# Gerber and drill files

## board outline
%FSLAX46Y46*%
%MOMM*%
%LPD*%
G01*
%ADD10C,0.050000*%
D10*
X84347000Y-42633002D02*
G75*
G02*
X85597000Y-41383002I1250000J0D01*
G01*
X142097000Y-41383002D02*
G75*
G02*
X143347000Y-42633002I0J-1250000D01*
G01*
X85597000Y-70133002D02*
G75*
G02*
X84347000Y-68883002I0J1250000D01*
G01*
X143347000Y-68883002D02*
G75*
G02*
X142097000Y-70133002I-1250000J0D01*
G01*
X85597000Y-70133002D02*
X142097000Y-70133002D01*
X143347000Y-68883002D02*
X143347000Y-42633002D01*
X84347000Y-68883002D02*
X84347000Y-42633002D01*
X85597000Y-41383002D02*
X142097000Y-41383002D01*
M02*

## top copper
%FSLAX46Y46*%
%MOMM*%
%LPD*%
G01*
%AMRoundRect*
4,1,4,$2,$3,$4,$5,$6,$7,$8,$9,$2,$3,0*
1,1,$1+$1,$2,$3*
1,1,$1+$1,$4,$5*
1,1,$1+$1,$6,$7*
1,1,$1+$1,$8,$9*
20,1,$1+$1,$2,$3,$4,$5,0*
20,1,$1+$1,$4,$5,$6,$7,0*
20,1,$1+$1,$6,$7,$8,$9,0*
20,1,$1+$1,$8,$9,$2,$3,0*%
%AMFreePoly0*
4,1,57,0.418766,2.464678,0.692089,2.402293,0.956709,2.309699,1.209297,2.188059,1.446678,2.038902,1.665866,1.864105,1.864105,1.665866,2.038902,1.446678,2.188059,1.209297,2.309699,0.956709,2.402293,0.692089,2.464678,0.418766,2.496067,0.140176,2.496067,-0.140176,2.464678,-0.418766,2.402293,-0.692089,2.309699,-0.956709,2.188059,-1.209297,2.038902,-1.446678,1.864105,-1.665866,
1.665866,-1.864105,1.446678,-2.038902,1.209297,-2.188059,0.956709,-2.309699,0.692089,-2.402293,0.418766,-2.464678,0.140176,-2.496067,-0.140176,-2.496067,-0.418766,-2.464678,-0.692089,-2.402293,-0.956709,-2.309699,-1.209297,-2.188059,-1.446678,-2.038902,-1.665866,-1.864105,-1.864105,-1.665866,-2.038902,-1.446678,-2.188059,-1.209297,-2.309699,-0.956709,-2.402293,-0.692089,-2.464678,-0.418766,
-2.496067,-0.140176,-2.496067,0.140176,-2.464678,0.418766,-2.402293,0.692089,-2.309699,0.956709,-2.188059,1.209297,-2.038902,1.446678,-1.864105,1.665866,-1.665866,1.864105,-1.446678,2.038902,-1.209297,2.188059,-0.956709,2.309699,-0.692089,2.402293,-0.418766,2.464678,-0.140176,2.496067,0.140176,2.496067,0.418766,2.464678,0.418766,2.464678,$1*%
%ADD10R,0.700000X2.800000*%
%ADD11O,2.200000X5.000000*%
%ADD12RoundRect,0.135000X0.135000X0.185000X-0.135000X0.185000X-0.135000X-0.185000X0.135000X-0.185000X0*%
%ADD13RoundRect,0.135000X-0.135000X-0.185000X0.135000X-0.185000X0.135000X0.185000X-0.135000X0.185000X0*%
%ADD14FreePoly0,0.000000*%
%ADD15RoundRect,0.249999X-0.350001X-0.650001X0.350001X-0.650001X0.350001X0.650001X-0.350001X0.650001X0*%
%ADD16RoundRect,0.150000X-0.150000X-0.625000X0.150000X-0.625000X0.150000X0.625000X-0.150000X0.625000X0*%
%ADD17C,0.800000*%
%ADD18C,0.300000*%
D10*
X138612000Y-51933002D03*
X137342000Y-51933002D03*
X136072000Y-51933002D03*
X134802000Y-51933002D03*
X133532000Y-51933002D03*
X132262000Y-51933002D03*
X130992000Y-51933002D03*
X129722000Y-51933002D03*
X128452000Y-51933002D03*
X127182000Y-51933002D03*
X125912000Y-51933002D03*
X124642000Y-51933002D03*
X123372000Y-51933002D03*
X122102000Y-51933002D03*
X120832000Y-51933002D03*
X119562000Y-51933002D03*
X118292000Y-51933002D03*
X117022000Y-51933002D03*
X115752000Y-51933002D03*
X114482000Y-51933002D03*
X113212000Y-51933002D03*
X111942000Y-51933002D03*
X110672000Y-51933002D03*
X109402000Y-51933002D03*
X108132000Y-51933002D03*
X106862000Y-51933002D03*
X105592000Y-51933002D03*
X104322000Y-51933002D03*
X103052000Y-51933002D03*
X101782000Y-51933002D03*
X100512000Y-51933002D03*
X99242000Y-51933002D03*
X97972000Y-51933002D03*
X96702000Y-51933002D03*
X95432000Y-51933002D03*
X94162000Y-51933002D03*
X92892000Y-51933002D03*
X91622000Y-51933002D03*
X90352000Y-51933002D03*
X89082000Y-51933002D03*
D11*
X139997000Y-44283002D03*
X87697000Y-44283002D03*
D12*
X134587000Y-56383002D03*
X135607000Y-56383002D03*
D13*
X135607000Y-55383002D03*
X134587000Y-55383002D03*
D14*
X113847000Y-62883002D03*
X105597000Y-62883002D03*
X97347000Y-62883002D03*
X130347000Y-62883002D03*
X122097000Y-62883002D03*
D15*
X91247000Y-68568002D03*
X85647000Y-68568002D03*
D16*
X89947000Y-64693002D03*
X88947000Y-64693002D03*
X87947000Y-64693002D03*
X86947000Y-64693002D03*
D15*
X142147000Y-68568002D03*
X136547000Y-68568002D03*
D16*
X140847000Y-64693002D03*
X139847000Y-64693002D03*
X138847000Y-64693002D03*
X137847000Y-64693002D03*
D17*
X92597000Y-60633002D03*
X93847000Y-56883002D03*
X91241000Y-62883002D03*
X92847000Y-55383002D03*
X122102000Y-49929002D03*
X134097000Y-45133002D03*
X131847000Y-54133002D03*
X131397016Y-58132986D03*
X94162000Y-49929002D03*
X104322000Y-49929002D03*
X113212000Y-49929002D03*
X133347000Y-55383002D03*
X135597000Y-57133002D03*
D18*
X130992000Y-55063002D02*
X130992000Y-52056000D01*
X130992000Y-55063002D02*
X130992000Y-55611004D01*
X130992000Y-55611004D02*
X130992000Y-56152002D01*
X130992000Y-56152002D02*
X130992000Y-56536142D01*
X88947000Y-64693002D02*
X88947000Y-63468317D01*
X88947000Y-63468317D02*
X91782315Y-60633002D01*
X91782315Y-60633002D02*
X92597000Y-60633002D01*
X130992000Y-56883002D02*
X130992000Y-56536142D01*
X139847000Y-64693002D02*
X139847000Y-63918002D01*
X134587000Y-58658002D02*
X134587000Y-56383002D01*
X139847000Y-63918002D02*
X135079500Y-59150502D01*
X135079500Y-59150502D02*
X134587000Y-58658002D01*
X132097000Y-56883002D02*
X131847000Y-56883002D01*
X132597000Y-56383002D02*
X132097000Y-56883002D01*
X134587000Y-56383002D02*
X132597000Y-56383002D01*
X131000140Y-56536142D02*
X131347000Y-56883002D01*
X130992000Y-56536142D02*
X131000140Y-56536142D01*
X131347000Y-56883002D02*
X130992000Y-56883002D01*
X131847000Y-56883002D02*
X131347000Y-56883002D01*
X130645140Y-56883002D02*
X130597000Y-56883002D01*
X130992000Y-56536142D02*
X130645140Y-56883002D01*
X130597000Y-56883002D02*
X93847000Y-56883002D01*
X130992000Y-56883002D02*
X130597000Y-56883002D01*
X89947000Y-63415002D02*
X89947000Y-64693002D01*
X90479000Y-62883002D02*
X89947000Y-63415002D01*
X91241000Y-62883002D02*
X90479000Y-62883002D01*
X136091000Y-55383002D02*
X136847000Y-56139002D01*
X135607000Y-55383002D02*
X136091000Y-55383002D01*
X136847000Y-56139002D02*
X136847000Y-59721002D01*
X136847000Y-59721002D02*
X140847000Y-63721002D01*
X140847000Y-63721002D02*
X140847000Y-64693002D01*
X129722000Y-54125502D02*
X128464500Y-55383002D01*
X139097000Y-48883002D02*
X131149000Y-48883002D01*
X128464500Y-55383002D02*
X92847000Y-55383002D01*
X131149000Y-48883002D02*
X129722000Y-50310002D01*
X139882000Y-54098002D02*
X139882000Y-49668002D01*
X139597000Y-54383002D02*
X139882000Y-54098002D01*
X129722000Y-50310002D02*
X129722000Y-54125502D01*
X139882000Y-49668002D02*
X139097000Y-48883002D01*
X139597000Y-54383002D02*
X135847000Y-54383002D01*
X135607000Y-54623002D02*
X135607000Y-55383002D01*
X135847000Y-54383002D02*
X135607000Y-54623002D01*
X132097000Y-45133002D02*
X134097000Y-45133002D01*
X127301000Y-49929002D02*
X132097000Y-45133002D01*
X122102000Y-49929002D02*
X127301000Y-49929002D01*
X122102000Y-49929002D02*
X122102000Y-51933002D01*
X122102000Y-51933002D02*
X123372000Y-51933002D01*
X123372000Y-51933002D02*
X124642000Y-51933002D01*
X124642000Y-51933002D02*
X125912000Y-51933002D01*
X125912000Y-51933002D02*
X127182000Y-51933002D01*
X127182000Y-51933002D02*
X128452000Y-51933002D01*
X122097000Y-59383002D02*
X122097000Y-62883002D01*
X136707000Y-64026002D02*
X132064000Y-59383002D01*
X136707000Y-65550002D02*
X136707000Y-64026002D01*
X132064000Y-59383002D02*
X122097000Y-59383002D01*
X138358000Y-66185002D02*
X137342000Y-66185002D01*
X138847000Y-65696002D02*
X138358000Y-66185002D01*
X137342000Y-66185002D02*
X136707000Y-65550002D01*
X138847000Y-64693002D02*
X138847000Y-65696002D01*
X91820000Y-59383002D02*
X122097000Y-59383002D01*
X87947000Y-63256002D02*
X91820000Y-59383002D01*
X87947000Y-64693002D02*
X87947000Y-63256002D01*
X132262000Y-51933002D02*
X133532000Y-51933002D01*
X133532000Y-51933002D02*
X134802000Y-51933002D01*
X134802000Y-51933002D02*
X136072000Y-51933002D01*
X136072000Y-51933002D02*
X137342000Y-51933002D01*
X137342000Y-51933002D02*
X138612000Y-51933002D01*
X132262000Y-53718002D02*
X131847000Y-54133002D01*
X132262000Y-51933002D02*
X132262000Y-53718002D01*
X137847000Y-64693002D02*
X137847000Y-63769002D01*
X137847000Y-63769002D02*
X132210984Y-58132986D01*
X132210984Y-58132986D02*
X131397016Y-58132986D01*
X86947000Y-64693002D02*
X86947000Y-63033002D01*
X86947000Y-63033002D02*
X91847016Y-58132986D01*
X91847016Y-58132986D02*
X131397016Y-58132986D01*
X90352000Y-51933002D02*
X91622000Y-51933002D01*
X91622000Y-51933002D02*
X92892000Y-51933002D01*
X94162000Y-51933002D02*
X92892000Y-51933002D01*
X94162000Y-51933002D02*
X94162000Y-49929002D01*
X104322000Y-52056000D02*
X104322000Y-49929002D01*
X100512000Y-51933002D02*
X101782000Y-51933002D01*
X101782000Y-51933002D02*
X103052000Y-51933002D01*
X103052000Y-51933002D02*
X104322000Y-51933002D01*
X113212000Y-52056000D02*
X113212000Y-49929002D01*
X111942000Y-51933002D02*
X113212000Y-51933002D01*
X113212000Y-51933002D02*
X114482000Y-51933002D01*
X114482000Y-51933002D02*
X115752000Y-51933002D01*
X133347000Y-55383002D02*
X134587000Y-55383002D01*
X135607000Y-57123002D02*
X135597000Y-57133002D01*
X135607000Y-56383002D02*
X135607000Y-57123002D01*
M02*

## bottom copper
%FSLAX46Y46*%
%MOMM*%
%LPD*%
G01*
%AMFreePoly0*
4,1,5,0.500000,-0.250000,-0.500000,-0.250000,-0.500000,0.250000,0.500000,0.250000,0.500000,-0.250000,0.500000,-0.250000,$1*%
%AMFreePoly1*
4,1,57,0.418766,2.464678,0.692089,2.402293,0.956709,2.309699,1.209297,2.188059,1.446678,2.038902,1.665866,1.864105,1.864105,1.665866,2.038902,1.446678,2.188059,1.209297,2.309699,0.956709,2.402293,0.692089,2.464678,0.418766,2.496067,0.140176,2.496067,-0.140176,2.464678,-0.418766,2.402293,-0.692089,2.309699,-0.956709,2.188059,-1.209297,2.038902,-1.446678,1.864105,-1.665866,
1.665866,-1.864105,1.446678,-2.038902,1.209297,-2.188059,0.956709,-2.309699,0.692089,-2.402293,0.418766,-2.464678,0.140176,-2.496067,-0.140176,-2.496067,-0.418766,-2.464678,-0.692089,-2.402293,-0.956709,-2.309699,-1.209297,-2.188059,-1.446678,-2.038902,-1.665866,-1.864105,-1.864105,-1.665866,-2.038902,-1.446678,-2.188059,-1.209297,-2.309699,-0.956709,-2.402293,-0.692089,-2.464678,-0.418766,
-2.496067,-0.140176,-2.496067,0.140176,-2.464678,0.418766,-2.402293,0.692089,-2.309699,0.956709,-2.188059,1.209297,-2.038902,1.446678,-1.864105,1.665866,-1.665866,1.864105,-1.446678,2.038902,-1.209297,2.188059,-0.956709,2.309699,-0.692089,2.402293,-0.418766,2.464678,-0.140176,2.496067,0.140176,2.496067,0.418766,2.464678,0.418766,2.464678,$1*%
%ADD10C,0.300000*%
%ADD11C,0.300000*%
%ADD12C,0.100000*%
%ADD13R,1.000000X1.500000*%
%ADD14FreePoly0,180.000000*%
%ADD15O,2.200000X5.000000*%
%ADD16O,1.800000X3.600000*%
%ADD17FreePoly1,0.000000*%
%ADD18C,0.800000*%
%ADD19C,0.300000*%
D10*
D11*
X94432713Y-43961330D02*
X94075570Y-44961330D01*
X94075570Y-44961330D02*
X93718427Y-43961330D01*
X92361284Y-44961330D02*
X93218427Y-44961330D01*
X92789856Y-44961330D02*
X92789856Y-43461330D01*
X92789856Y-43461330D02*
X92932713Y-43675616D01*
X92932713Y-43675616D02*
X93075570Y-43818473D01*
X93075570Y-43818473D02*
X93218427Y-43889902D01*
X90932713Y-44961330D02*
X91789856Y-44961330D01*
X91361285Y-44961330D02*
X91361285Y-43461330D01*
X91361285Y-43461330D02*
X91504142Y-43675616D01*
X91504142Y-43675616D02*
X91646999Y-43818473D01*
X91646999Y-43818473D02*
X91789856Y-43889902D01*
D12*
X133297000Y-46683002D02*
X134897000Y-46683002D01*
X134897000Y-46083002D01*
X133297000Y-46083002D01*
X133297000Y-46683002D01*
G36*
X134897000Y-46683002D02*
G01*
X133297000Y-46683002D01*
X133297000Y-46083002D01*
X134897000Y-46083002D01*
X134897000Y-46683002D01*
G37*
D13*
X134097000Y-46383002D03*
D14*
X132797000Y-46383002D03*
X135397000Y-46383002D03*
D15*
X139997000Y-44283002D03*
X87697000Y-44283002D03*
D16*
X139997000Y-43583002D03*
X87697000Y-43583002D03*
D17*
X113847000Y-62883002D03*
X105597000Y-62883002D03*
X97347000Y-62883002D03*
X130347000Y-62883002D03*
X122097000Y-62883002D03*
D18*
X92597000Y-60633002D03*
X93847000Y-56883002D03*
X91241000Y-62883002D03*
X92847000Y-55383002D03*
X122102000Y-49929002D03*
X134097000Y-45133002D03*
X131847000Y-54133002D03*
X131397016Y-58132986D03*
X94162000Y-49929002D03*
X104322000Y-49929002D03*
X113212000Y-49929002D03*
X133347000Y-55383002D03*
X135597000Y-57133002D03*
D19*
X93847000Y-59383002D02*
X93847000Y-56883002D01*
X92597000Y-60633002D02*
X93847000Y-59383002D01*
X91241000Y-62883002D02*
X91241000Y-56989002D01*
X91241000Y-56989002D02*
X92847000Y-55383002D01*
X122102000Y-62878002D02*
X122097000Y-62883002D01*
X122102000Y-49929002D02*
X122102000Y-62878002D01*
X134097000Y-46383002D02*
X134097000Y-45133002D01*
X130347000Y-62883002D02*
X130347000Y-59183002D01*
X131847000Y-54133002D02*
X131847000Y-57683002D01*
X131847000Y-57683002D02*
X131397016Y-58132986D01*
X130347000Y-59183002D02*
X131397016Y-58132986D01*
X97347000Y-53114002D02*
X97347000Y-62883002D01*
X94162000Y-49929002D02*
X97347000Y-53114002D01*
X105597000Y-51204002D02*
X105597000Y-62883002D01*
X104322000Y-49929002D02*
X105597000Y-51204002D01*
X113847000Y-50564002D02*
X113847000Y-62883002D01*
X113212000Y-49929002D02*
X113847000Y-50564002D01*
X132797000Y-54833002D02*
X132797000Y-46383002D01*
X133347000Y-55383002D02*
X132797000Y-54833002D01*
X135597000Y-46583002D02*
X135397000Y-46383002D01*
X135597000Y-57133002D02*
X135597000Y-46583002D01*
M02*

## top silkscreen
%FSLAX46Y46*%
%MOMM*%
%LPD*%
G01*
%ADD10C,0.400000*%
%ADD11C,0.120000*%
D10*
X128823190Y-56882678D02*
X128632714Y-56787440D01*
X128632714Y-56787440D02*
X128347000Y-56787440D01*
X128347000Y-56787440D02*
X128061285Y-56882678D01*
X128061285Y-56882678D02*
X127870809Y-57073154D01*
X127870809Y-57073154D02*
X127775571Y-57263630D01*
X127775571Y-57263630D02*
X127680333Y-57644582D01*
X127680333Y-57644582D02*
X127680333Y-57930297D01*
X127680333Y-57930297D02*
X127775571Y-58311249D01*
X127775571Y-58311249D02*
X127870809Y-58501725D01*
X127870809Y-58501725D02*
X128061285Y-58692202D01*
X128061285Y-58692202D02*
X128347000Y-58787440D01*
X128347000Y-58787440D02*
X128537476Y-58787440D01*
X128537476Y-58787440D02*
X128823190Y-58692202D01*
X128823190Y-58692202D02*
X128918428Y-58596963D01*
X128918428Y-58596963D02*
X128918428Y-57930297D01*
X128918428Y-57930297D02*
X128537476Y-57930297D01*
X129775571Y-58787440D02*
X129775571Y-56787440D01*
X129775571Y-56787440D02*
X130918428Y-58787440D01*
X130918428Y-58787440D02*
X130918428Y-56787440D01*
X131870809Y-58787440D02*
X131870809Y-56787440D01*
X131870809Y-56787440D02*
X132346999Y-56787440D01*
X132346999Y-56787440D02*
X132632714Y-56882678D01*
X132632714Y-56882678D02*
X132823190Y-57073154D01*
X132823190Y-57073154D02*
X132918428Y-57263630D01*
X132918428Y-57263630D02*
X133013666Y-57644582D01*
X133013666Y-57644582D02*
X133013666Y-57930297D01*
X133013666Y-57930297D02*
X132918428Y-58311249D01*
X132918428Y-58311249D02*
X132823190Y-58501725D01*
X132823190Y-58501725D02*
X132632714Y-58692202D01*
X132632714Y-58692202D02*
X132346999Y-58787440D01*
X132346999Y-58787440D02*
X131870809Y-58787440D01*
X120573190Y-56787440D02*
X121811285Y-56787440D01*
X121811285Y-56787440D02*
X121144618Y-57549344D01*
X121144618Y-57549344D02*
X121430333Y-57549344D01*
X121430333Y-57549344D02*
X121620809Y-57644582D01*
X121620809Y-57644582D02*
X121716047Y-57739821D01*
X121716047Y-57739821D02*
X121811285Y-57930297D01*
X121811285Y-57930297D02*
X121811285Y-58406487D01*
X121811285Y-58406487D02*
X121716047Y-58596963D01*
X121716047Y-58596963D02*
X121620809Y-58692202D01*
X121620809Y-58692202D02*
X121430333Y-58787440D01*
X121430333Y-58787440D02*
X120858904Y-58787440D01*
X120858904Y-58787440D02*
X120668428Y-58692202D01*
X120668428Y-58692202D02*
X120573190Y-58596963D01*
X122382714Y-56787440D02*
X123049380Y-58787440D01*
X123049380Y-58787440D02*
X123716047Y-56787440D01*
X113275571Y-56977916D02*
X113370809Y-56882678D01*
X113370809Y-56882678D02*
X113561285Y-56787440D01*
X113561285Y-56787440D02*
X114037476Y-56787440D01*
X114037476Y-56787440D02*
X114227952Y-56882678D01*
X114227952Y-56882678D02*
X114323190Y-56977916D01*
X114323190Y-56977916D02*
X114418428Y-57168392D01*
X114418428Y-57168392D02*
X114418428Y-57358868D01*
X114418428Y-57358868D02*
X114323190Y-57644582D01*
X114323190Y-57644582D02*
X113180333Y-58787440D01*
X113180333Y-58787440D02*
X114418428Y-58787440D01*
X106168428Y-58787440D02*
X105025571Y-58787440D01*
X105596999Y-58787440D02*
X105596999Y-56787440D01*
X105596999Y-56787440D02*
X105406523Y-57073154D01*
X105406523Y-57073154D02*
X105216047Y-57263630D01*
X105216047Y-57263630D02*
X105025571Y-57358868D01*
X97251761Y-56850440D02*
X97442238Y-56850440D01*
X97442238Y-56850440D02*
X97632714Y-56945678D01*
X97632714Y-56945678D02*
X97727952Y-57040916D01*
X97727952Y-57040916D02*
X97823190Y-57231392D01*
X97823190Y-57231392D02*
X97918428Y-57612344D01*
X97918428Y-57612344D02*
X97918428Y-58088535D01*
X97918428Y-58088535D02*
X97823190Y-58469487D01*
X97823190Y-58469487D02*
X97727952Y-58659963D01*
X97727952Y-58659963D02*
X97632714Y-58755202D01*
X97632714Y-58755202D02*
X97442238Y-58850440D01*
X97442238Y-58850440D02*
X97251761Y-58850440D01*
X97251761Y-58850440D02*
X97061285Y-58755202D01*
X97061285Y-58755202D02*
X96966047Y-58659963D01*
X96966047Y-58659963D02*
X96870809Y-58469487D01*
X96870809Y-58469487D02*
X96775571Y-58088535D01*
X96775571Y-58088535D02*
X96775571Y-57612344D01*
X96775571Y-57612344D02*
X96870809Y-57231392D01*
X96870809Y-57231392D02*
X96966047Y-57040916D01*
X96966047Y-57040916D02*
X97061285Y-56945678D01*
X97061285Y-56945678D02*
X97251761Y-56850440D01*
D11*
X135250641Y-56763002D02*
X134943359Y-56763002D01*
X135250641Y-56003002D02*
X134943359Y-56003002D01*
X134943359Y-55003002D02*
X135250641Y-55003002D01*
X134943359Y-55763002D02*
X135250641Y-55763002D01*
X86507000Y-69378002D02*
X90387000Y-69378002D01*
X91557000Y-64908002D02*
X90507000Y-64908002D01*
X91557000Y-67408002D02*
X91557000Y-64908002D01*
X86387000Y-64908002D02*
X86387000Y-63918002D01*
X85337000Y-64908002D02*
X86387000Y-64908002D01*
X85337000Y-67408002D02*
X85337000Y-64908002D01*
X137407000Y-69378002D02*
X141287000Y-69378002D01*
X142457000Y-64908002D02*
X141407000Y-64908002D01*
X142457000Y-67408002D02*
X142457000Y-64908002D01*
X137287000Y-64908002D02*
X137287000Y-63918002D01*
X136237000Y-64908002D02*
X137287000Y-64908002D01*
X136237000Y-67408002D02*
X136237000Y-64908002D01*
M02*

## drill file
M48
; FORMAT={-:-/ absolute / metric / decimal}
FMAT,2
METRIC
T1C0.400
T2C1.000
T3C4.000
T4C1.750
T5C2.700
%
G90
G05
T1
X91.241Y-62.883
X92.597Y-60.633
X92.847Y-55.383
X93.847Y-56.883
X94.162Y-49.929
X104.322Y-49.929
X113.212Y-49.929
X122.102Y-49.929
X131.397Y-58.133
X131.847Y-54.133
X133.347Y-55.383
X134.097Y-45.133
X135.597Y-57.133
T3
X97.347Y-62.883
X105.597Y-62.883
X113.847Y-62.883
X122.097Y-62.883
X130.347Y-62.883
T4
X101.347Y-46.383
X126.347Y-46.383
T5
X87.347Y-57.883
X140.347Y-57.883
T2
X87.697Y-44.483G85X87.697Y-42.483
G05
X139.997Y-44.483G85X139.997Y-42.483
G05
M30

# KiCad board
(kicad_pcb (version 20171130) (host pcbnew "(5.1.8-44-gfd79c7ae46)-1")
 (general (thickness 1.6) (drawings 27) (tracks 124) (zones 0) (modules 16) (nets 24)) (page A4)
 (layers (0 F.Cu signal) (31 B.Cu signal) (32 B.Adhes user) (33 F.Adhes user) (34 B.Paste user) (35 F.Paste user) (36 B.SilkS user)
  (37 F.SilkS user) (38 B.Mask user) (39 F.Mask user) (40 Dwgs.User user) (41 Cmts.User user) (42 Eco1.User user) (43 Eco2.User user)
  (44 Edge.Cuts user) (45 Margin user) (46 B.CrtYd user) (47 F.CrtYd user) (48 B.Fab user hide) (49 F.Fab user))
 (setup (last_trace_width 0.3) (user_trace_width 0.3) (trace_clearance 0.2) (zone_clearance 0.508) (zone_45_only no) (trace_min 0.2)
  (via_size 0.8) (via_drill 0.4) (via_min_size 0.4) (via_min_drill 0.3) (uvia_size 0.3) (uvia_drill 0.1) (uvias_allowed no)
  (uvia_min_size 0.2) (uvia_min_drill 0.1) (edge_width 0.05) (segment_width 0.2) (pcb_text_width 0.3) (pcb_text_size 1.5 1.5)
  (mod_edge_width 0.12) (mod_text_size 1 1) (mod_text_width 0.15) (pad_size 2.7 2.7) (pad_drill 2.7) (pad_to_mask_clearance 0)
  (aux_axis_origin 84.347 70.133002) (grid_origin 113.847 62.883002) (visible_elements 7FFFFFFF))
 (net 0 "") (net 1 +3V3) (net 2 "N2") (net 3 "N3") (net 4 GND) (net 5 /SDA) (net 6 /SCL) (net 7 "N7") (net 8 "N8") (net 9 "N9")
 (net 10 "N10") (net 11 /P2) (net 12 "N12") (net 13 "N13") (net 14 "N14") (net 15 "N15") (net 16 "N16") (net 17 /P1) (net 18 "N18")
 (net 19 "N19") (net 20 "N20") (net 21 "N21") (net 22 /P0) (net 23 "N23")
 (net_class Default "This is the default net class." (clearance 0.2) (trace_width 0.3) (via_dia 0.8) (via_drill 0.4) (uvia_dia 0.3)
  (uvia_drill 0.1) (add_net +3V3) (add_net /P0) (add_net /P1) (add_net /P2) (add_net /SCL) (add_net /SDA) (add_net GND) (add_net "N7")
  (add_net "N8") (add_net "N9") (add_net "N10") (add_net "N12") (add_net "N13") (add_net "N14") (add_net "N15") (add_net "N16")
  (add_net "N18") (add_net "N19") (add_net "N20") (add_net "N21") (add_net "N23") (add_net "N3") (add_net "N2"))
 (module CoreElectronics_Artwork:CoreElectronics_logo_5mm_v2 (layer B.Cu) (at 140.247 66.883002 180)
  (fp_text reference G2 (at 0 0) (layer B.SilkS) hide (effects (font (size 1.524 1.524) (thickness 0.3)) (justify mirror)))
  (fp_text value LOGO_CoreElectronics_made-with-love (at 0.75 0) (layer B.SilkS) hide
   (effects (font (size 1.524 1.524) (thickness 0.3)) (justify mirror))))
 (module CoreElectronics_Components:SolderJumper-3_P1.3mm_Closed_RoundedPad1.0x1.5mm (layer B.Cu) (at 134.097 46.383002 180)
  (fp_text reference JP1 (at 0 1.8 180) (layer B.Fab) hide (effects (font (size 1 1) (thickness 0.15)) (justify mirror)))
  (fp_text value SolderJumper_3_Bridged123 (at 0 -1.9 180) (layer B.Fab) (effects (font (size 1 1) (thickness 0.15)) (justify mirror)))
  (fp_poly (pts (xy 0.8 -0.3) (xy -0.8 -0.3) (xy -0.8 0.3) (xy 0.8 0.3)) (layer B.Cu) (width 0.1))
  (pad 2 smd rect (at 0 0 180) (size 1 1.5) (layers B.Cu B.Mask) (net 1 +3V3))
  (pad 3 smd custom (at 1.3 0 180) (size 1 0.5) (layers B.Cu B.Mask) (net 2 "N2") (zone_connect 2)
   (options (clearance outline) (anchor rect)) (primitives))
  (pad 1 smd custom (at -1.3 0 180) (size 1 0.5) (layers B.Cu B.Mask) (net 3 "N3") (zone_connect 2)
   (options (clearance outline) (anchor rect)) (primitives)))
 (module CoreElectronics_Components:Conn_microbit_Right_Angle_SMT (layer F.Cu) (at 113.847 46.383002 180)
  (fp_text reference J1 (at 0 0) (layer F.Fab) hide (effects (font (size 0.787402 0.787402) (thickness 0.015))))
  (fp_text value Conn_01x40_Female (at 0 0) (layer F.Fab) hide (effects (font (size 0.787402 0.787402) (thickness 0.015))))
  (pad 1 smd rect (at -24.765 -5.55 180) (size 0.7 2.8) (layers F.Cu F.Paste F.Mask) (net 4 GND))
  (pad 2 smd rect (at -23.495 -5.55 180) (size 0.7 2.8) (layers F.Cu F.Paste F.Mask) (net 4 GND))
  (pad 3 smd rect (at -22.225 -5.55 180) (size 0.7 2.8) (layers F.Cu F.Paste F.Mask) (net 4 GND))
  (pad 4 smd rect (at -20.955 -5.55 180) (size 0.7 2.8) (layers F.Cu F.Paste F.Mask) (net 4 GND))
  (pad 5 smd rect (at -19.685 -5.55 180) (size 0.7 2.8) (layers F.Cu F.Paste F.Mask) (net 4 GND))
  (pad 6 smd rect (at -18.415 -5.55 180) (size 0.7 2.8) (layers F.Cu F.Paste F.Mask) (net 4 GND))
  (pad 7 smd rect (at -17.145 -5.55 180) (size 0.7 2.8) (layers F.Cu F.Paste F.Mask) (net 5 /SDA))
  (pad 8 smd rect (at -15.875 -5.55 180) (size 0.7 2.8) (layers F.Cu F.Paste F.Mask) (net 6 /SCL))
  (pad 9 smd rect (at -14.605 -5.55 180) (size 0.7 2.8) (layers F.Cu F.Paste F.Mask) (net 1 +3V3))
  (pad 10 smd rect (at -13.335 -5.55 180) (size 0.7 2.8) (layers F.Cu F.Paste F.Mask) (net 1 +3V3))
  (pad 11 smd rect (at -12.065 -5.55 180) (size 0.7 2.8) (layers F.Cu F.Paste F.Mask) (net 1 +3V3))
  (pad 12 smd rect (at -10.795 -5.55 180) (size 0.7 2.8) (layers F.Cu F.Paste F.Mask) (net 1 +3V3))
  (pad 13 smd rect (at -9.525 -5.55 180) (size 0.7 2.8) (layers F.Cu F.Paste F.Mask) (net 1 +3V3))
  (pad 14 smd rect (at -8.255 -5.55 180) (size 0.7 2.8) (layers F.Cu F.Paste F.Mask) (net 1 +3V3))
  (pad 15 smd rect (at -6.985 -5.55 180) (size 0.7 2.8) (layers F.Cu F.Paste F.Mask) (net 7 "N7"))
  (pad 16 smd rect (at -5.715 -5.55 180) (size 0.7 2.8) (layers F.Cu F.Paste F.Mask) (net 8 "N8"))
  (pad 17 smd rect (at -4.445 -5.55 180) (size 0.7 2.8) (layers F.Cu F.Paste F.Mask) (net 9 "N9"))
  (pad 18 smd rect (at -3.175 -5.55 180) (size 0.7 2.8) (layers F.Cu F.Paste F.Mask) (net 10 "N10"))
  (pad 19 smd rect (at -1.905 -5.55 180) (size 0.7 2.8) (layers F.Cu F.Paste F.Mask) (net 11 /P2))
  (pad 20 smd rect (at -0.635 -5.55 180) (size 0.7 2.8) (layers F.Cu F.Paste F.Mask) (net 11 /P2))
  (pad 21 smd rect (at 0.635 -5.55 180) (size 0.7 2.8) (layers F.Cu F.Paste F.Mask) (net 11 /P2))
  (pad 22 smd rect (at 1.905 -5.55 180) (size 0.7 2.8) (layers F.Cu F.Paste F.Mask) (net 11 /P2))
  (pad 23 smd rect (at 3.175 -5.55 180) (size 0.7 2.8) (layers F.Cu F.Paste F.Mask) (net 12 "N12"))
  (pad 24 smd rect (at 4.445 -5.55 180) (size 0.7 2.8) (layers F.Cu F.Paste F.Mask) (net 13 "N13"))
  (pad 25 smd rect (at 5.715 -5.55 180) (size 0.7 2.8) (layers F.Cu F.Paste F.Mask) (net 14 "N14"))
  (pad 26 smd rect (at 6.985 -5.55 180) (size 0.7 2.8) (layers F.Cu F.Paste F.Mask) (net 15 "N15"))
  (pad 27 smd rect (at 8.255 -5.55 180) (size 0.7 2.8) (layers F.Cu F.Paste F.Mask) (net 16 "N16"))
  (pad 28 smd rect (at 9.525 -5.55 180) (size 0.7 2.8) (layers F.Cu F.Paste F.Mask) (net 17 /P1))
  (pad 29 smd rect (at 10.795 -5.55 180) (size 0.7 2.8) (layers F.Cu F.Paste F.Mask) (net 17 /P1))
  (pad 30 smd rect (at 12.065 -5.55 180) (size 0.7 2.8) (layers F.Cu F.Paste F.Mask) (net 17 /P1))
  (pad 31 smd rect (at 13.335 -5.55 180) (size 0.7 2.8) (layers F.Cu F.Paste F.Mask) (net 17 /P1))
  (pad 32 smd rect (at 14.605 -5.55 180) (size 0.7 2.8) (layers F.Cu F.Paste F.Mask) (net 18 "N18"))
  (pad 33 smd rect (at 15.875 -5.55 180) (size 0.7 2.8) (layers F.Cu F.Paste F.Mask) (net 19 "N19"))
  (pad 34 smd rect (at 17.145 -5.55 180) (size 0.7 2.8) (layers F.Cu F.Paste F.Mask) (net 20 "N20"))
  (pad 35 smd rect (at 18.415 -5.55 180) (size 0.7 2.8) (layers F.Cu F.Paste F.Mask) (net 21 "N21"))
  (pad 36 smd rect (at 19.685 -5.55 180) (size 0.7 2.8) (layers F.Cu F.Paste F.Mask) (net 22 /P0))
  (pad 37 smd rect (at 20.955 -5.55 180) (size 0.7 2.8) (layers F.Cu F.Paste F.Mask) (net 22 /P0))
  (pad 38 smd rect (at 22.225 -5.55 180) (size 0.7 2.8) (layers F.Cu F.Paste F.Mask) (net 22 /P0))
  (pad 39 smd rect (at 23.495 -5.55 180) (size 0.7 2.8) (layers F.Cu F.Paste F.Mask) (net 22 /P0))
  (pad 40 smd rect (at 24.765 -5.55 180) (size 0.7 2.8) (layers F.Cu F.Paste F.Mask) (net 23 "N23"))
  (pad None np_thru_hole circle (at -12.5 0 180) (size 1.75 1.75) (drill 1.75) (layers *.Cu *.Mask))
  (pad None np_thru_hole circle (at 12.5 0 180) (size 1.75 1.75) (drill 1.75) (layers *.Cu *.Mask))
  (pad MP thru_hole oval (at -26.15 2.9 180) (size 2.2 5) (drill oval 1 3 (offset 0 -0.8)) (layers F.Cu F.Paste F.Mask))
  (pad MP thru_hole oval (at 26.15 2.9 180) (size 2.2 5) (drill oval 1 3 (offset 0 -0.8)) (layers F.Cu F.Paste F.Mask))
  (pad MP smd oval (at -26.15 2.8 180) (size 1.8 3.6) (layers B.Cu B.Mask))
  (pad MP smd oval (at 26.15 2.8 180) (size 1.8 3.6) (layers B.Cu B.Mask)))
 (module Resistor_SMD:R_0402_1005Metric (layer F.Cu) (at 135.097 56.383002 180)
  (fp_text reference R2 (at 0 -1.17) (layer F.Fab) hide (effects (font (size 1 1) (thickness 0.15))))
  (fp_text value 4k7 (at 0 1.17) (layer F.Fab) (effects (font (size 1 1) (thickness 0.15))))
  (fp_line (start -0.153641 -0.38) (end 0.153641 -0.38) (layer F.SilkS) (width 0.12))
  (fp_line (start -0.153641 0.38) (end 0.153641 0.38) (layer F.SilkS) (width 0.12))
  (pad 2 smd roundrect (at 0.51 0 180) (size 0.54 0.64) (layers F.Cu F.Paste F.Mask) (roundrect_rratio 0.25) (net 5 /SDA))
  (pad 1 smd roundrect (at -0.51 0 180) (size 0.54 0.64) (layers F.Cu F.Paste F.Mask) (roundrect_rratio 0.25) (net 3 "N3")))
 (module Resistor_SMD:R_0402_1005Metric (layer F.Cu) (at 135.097 55.383002)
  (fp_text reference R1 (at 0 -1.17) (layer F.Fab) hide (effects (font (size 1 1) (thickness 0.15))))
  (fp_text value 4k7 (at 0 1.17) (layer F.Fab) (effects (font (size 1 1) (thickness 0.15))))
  (fp_line (start -0.153641 -0.38) (end 0.153641 -0.38) (layer F.SilkS) (width 0.12))
  (fp_line (start -0.153641 0.38) (end 0.153641 0.38) (layer F.SilkS) (width 0.12))
  (pad 2 smd roundrect (at 0.51 0) (size 0.54 0.64) (layers F.Cu F.Paste F.Mask) (roundrect_rratio 0.25) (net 6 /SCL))
  (pad 1 smd roundrect (at -0.51 0) (size 0.54 0.64) (layers F.Cu F.Paste F.Mask) (roundrect_rratio 0.25) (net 2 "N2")))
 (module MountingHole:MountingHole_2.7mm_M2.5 (layer F.Cu) (at 87.347 57.883002)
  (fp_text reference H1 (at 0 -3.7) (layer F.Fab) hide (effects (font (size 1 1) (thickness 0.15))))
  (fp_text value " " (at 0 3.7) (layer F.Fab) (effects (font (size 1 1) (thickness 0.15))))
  (pad "" np_thru_hole circle (at 0 0) (size 2.7 2.7) (drill 2.7) (layers *.Cu *.Mask) (clearance 1.35)))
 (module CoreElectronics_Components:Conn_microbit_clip (layer F.Cu) (at 113.847 62.883002)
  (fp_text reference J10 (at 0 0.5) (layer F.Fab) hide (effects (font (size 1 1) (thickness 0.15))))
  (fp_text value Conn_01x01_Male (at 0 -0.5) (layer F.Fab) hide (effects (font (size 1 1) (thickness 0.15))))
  (pad 1 thru_hole custom (at 0 0) (size 5 5) (drill 4) (layers *.Cu *.Mask) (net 11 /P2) (zone_connect 0)
   (options (clearance outline) (anchor circle)) (primitives)))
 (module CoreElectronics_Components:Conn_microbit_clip (layer F.Cu) (at 105.597 62.883002)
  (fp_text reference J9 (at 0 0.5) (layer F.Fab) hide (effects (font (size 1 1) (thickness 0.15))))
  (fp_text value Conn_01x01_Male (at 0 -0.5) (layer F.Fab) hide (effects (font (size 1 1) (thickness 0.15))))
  (pad 1 thru_hole custom (at 0 0) (size 5 5) (drill 4) (layers *.Cu *.Mask) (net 17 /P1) (zone_connect 0)
   (options (clearance outline) (anchor circle)) (primitives)))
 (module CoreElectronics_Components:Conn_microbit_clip (layer F.Cu) (at 97.347 62.883002)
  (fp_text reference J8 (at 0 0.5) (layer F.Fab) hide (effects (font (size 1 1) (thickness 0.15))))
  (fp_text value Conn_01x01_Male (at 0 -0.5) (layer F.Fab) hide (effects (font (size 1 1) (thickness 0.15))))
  (pad 1 thru_hole custom (at 0 0) (size 5 5) (drill 4) (layers *.Cu *.Mask) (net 22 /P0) (zone_connect 0)
   (options (clearance outline) (anchor circle)) (primitives)))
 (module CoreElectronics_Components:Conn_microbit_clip (layer F.Cu) (at 130.347 62.883002)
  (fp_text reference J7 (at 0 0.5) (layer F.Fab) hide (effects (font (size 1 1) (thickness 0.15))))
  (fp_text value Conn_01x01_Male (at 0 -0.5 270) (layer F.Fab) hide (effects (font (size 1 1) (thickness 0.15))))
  (pad 1 thru_hole custom (at 0 0) (size 5 5) (drill 4) (layers *.Cu *.Mask) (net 4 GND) (zone_connect 0)
   (options (clearance outline) (anchor circle)) (primitives)))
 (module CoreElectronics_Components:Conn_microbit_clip (layer F.Cu) (at 122.097 62.883002)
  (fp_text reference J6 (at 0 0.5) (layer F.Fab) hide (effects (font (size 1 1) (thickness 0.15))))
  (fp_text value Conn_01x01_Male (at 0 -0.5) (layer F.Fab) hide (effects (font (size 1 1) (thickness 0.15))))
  (pad 1 thru_hole custom (at 0 0) (size 5 5) (drill 4) (layers *.Cu *.Mask) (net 1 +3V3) (zone_connect 0)
   (options (clearance outline) (anchor circle)) (primitives)))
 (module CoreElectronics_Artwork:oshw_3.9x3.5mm (layer B.Cu) (at 87.847 67.269002 180)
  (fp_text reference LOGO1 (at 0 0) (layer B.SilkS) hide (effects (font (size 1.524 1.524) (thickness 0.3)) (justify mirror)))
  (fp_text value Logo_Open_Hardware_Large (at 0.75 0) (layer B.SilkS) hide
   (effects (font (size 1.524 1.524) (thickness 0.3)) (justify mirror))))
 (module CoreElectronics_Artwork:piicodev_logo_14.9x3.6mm (layer B.Cu) (at 113.847 45.386001 180)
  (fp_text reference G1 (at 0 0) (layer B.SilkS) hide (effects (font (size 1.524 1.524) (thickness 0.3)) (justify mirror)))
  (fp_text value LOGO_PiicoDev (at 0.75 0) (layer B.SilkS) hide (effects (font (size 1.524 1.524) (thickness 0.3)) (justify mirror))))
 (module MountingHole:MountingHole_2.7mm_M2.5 (layer F.Cu) (at 140.347 57.883002)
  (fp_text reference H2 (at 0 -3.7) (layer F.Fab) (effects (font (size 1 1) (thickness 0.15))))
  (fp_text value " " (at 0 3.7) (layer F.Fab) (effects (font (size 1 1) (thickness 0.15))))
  (pad "" np_thru_hole circle (at 0 0) (size 2.7 2.7) (drill 2.7) (layers *.Cu *.Mask) (clearance 1.35)))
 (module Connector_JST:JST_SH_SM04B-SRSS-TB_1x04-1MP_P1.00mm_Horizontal (layer F.Cu) (at 88.447 66.693002)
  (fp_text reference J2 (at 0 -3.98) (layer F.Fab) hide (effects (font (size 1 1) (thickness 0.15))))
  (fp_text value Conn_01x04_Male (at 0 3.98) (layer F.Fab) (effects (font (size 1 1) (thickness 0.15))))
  (fp_line (start -1.94 2.685) (end 1.94 2.685) (layer F.SilkS) (width 0.12))
  (fp_line (start 3.11 -1.785) (end 2.06 -1.785) (layer F.SilkS) (width 0.12))
  (fp_line (start 3.11 0.715) (end 3.11 -1.785) (layer F.SilkS) (width 0.12))
  (fp_line (start -2.06 -1.785) (end -2.06 -2.775) (layer F.SilkS) (width 0.12))
  (fp_line (start -3.11 -1.785) (end -2.06 -1.785) (layer F.SilkS) (width 0.12))
  (fp_line (start -3.11 0.715) (end -3.11 -1.785) (layer F.SilkS) (width 0.12))
  (pad MP smd roundrect (at 2.8 1.875) (size 1.2 1.8) (layers F.Cu F.Paste F.Mask) (roundrect_rratio 0.2083325))
  (pad MP smd roundrect (at -2.8 1.875) (size 1.2 1.8) (layers F.Cu F.Paste F.Mask) (roundrect_rratio 0.2083325))
  (pad 4 smd roundrect (at 1.5 -2) (size 0.6 1.55) (layers F.Cu F.Paste F.Mask) (roundrect_rratio 0.25) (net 6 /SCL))
  (pad 3 smd roundrect (at 0.5 -2) (size 0.6 1.55) (layers F.Cu F.Paste F.Mask) (roundrect_rratio 0.25) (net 5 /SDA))
  (pad 2 smd roundrect (at -0.5 -2) (size 0.6 1.55) (layers F.Cu F.Paste F.Mask) (roundrect_rratio 0.25) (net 1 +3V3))
  (pad 1 smd roundrect (at -1.5 -2) (size 0.6 1.55) (layers F.Cu F.Paste F.Mask) (roundrect_rratio 0.25) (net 4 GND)))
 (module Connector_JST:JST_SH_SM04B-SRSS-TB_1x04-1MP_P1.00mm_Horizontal (layer F.Cu) (at 139.347 66.693002)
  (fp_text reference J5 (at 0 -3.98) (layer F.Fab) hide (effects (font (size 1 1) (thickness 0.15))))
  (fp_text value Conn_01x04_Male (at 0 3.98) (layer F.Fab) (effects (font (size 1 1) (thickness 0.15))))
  (fp_line (start -1.94 2.685) (end 1.94 2.685) (layer F.SilkS) (width 0.12))
  (fp_line (start 3.11 -1.785) (end 2.06 -1.785) (layer F.SilkS) (width 0.12))
  (fp_line (start 3.11 0.715) (end 3.11 -1.785) (layer F.SilkS) (width 0.12))
  (fp_line (start -2.06 -1.785) (end -2.06 -2.775) (layer F.SilkS) (width 0.12))
  (fp_line (start -3.11 -1.785) (end -2.06 -1.785) (layer F.SilkS) (width 0.12))
  (fp_line (start -3.11 0.715) (end -3.11 -1.785) (layer F.SilkS) (width 0.12))
  (pad MP smd roundrect (at 2.8 1.875) (size 1.2 1.8) (layers F.Cu F.Paste F.Mask) (roundrect_rratio 0.2083325))
  (pad MP smd roundrect (at -2.8 1.875) (size 1.2 1.8) (layers F.Cu F.Paste F.Mask) (roundrect_rratio 0.2083325))
  (pad 4 smd roundrect (at 1.5 -2) (size 0.6 1.55) (layers F.Cu F.Paste F.Mask) (roundrect_rratio 0.25) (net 6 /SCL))
  (pad 3 smd roundrect (at 0.5 -2) (size 0.6 1.55) (layers F.Cu F.Paste F.Mask) (roundrect_rratio 0.25) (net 5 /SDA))
  (pad 2 smd roundrect (at -0.5 -2) (size 0.6 1.55) (layers F.Cu F.Paste F.Mask) (roundrect_rratio 0.25) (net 1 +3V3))
  (pad 1 smd roundrect (at -1.5 -2) (size 0.6 1.55) (layers F.Cu F.Paste F.Mask) (roundrect_rratio 0.25) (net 4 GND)))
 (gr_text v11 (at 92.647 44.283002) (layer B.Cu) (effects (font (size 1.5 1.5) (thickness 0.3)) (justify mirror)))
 (gr_arc (start 85.597 42.633002) (end 85.597 41.383002) (angle -90) (layer Edge.Cuts) (width 0.05))
 (gr_arc (start 142.097 42.633002) (end 143.347 42.633002) (angle -90) (layer Edge.Cuts) (width 0.05))
 (gr_arc (start 85.597 68.883002) (end 84.347 68.883002) (angle -90) (layer Edge.Cuts) (width 0.05))
 (gr_arc (start 142.097 68.883002) (end 142.097 70.133002) (angle -90) (layer Edge.Cuts) (width 0.05))
 (gr_line (start 85.597 70.133002) (end 142.097 70.133002) (layer Edge.Cuts) (width 0.05))
 (gr_line (start 143.347 68.883002) (end 143.347 42.633002) (layer Edge.Cuts) (width 0.05))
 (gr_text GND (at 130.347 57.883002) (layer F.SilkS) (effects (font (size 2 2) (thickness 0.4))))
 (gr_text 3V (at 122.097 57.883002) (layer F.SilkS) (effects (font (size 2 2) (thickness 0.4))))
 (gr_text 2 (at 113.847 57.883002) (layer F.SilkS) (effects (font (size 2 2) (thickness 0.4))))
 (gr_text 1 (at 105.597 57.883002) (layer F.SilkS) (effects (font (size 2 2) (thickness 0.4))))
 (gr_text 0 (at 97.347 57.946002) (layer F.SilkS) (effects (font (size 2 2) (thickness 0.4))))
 (gr_line (start 84.347 68.883002) (end 84.347 42.633002) (layer Edge.Cuts) (width 0.05))
 (gr_line (start 85.597 41.383002) (end 142.097 41.383002) (layer Edge.Cuts) (width 0.05))
 (segment (start 130.992 55.063002) (end 130.992 52.056) (width 0.3) (layer F.Cu) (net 5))
 (segment (start 130.992 55.063002) (end 130.992 55.611004) (width 0.3) (layer F.Cu) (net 5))
 (segment (start 130.992 55.611004) (end 130.992 56.152002) (width 0.3) (layer F.Cu) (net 5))
 (segment (start 130.992 56.152002) (end 130.992 56.536142) (width 0.3) (layer F.Cu) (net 5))
 (via (at 92.597 60.633002) (size 0.8) (drill 0.4) (layers F.Cu B.Cu) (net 5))
 (segment (start 88.947 64.693002) (end 88.947 63.468317) (width 0.3) (layer F.Cu) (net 5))
 (segment (start 88.947 63.468317) (end 91.782315 60.633002) (width 0.3) (layer F.Cu) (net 5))
 (segment (start 91.782315 60.633002) (end 92.597 60.633002) (width 0.3) (layer F.Cu) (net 5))
 (segment (start 93.847 59.383002) (end 93.847 56.883002) (width 0.3) (layer B.Cu) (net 5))
 (segment (start 92.597 60.633002) (end 93.847 59.383002) (width 0.3) (layer B.Cu) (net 5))
 (via (at 93.847 56.883002) (size 0.8) (drill 0.4) (layers F.Cu B.Cu) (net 5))
 (segment (start 130.992 56.883002) (end 130.992 56.536142) (width 0.3) (layer F.Cu) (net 5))
 (segment (start 139.847 64.693002) (end 139.847 63.918002) (width 0.3) (layer F.Cu) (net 5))
 (segment (start 134.587 58.658002) (end 134.587 56.383002) (width 0.3) (layer F.Cu) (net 5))
 (segment (start 139.847 63.918002) (end 135.0795 59.150502) (width 0.3) (layer F.Cu) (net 5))
 (segment (start 135.0795 59.150502) (end 134.587 58.658002) (width 0.3) (layer F.Cu) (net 5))
 (segment (start 132.097 56.883002) (end 131.847 56.883002) (width 0.3) (layer F.Cu) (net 5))
 (segment (start 132.597 56.383002) (end 132.097 56.883002) (width 0.3) (layer F.Cu) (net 5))
 (segment (start 134.587 56.383002) (end 132.597 56.383002) (width 0.3) (layer F.Cu) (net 5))
 (segment (start 131.00014 56.536142) (end 131.347 56.883002) (width 0.3) (layer F.Cu) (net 5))
 (segment (start 130.992 56.536142) (end 131.00014 56.536142) (width 0.3) (layer F.Cu) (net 5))
 (segment (start 131.347 56.883002) (end 130.992 56.883002) (width 0.3) (layer F.Cu) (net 5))
 (segment (start 131.847 56.883002) (end 131.347 56.883002) (width 0.3) (layer F.Cu) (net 5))
 (segment (start 130.64514 56.883002) (end 130.597 56.883002) (width 0.3) (layer F.Cu) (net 5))
 (segment (start 130.992 56.536142) (end 130.64514 56.883002) (width 0.3) (layer F.Cu) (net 5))
 (segment (start 130.597 56.883002) (end 93.847 56.883002) (width 0.3) (layer F.Cu) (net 5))
 (segment (start 130.992 56.883002) (end 130.597 56.883002) (width 0.3) (layer F.Cu) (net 5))
 (via (at 91.241 62.883002) (size 0.8) (drill 0.4) (layers F.Cu B.Cu) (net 6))
 (segment (start 89.947 63.415002) (end 89.947 64.693002) (width 0.3) (layer F.Cu) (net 6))
 (segment (start 90.479 62.883002) (end 89.947 63.415002) (width 0.3) (layer F.Cu) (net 6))
 (segment (start 91.241 62.883002) (end 90.479 62.883002) (width 0.3) (layer F.Cu) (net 6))
 (segment (start 136.091 55.383002) (end 136.847 56.139002) (width 0.3) (layer F.Cu) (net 6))
 (segment (start 135.607 55.383002) (end 136.091 55.383002) (width 0.3) (layer F.Cu) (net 6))
 (via (at 92.847 55.383002) (size 0.8) (drill 0.4) (layers F.Cu B.Cu) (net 6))
 (segment (start 91.241 62.883002) (end 91.241 56.989002) (width 0.3) (layer B.Cu) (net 6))
 (segment (start 91.241 56.989002) (end 92.847 55.383002) (width 0.3) (layer B.Cu) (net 6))
 (segment (start 136.847 56.139002) (end 136.847 59.721002) (width 0.3) (layer F.Cu) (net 6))
 (segment (start 136.847 59.721002) (end 140.847 63.721002) (width 0.3) (layer F.Cu) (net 6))
 (segment (start 140.847 63.721002) (end 140.847 64.693002) (width 0.3) (layer F.Cu) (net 6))
 (segment (start 129.722 54.125502) (end 128.4645 55.383002) (width 0.3) (layer F.Cu) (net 6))
 (segment (start 139.097 48.883002) (end 131.149 48.883002) (width 0.3) (layer F.Cu) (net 6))
 (segment (start 128.4645 55.383002) (end 92.847 55.383002) (width 0.3) (layer F.Cu) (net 6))
 (segment (start 131.149 48.883002) (end 129.722 50.310002) (width 0.3) (layer F.Cu) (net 6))
 (segment (start 139.882 54.098002) (end 139.882 49.668002) (width 0.3) (layer F.Cu) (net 6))
 (segment (start 139.597 54.383002) (end 139.882 54.098002) (width 0.3) (layer F.Cu) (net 6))
 (segment (start 129.722 50.310002) (end 129.722 54.125502) (width 0.3) (layer F.Cu) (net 6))
 (segment (start 139.882 49.668002) (end 139.097 48.883002) (width 0.3) (layer F.Cu) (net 6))
 (segment (start 139.597 54.383002) (end 135.847 54.383002) (width 0.3) (layer F.Cu) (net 6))
 (segment (start 135.607 54.623002) (end 135.607 55.383002) (width 0.3) (layer F.Cu) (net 6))
 (segment (start 135.847 54.383002) (end 135.607 54.623002) (width 0.3) (layer F.Cu) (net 6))
 (via (at 122.102 49.929002) (size 0.8) (drill 0.4) (layers F.Cu B.Cu) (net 1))
 (segment (start 122.102 62.878002) (end 122.097 62.883002) (width 0.3) (layer B.Cu) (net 1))
 (segment (start 122.102 49.929002) (end 122.102 62.878002) (width 0.3) (layer B.Cu) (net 1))
 (segment (start 134.097 46.383002) (end 134.097 45.133002) (width 0.3) (layer B.Cu) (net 1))
 (via (at 134.097 45.133002) (size 0.8) (drill 0.4) (layers F.Cu B.Cu) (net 1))
 (segment (start 132.097 45.133002) (end 134.097 45.133002) (width 0.3) (layer F.Cu) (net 1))
 (segment (start 127.301 49.929002) (end 132.097 45.133002) (width 0.3) (layer F.Cu) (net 1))
 (segment (start 122.102 49.929002) (end 127.301 49.929002) (width 0.3) (layer F.Cu) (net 1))
 (segment (start 122.102 49.929002) (end 122.102 51.933002) (width 0.3) (layer F.Cu) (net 1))
 (segment (start 122.102 51.933002) (end 123.372 51.933002) (width 0.3) (layer F.Cu) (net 1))
 (segment (start 123.372 51.933002) (end 124.642 51.933002) (width 0.3) (layer F.Cu) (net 1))
 (segment (start 124.642 51.933002) (end 125.912 51.933002) (width 0.3) (layer F.Cu) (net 1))
 (segment (start 125.912 51.933002) (end 127.182 51.933002) (width 0.3) (layer F.Cu) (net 1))
 (segment (start 127.182 51.933002) (end 128.452 51.933002) (width 0.3) (layer F.Cu) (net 1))
 (segment (start 122.097 59.383002) (end 122.097 62.883002) (width 0.3) (layer F.Cu) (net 1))
 (segment (start 136.707 64.026002) (end 132.064 59.383002) (width 0.3) (layer F.Cu) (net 1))
 (segment (start 136.707 65.550002) (end 136.707 64.026002) (width 0.3) (layer F.Cu) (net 1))
 (segment (start 132.064 59.383002) (end 122.097 59.383002) (width 0.3) (layer F.Cu) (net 1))
 (segment (start 138.358 66.185002) (end 137.342 66.185002) (width 0.3) (layer F.Cu) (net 1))
 (segment (start 138.847 65.696002) (end 138.358 66.185002) (width 0.3) (layer F.Cu) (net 1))
 (segment (start 137.342 66.185002) (end 136.707 65.550002) (width 0.3) (layer F.Cu) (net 1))
 (segment (start 138.847 64.693002) (end 138.847 65.696002) (width 0.3) (layer F.Cu) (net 1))
 (segment (start 91.82 59.383002) (end 122.097 59.383002) (width 0.3) (layer F.Cu) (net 1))
 (segment (start 87.947 63.256002) (end 91.82 59.383002) (width 0.3) (layer F.Cu) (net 1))
 (segment (start 87.947 64.693002) (end 87.947 63.256002) (width 0.3) (layer F.Cu) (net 1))
 (via (at 131.847 54.133002) (size 0.8) (drill 0.4) (layers F.Cu B.Cu) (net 4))
 (segment (start 132.262 51.933002) (end 133.532 51.933002) (width 0.3) (layer F.Cu) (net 4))
 (segment (start 133.532 51.933002) (end 134.802 51.933002) (width 0.3) (layer F.Cu) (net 4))
 (segment (start 134.802 51.933002) (end 136.072 51.933002) (width 0.3) (layer F.Cu) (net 4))
 (segment (start 136.072 51.933002) (end 137.342 51.933002) (width 0.3) (layer F.Cu) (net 4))
 (segment (start 137.342 51.933002) (end 138.612 51.933002) (width 0.3) (layer F.Cu) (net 4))
 (segment (start 132.262 53.718002) (end 131.847 54.133002) (width 0.3) (layer F.Cu) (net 4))
 (segment (start 132.262 51.933002) (end 132.262 53.718002) (width 0.3) (layer F.Cu) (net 4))
 (segment (start 130.347 62.883002) (end 130.347 59.183002) (width 0.3) (layer B.Cu) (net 4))
 (segment (start 137.847 64.693002) (end 137.847 63.769002) (width 0.3) (layer F.Cu) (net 4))
 (segment (start 131.847 54.133002) (end 131.847 57.683002) (width 0.3) (layer B.Cu) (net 4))
 (segment (start 131.847 57.683002) (end 131.397016 58.132986) (width 0.3) (layer B.Cu) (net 4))
 (segment (start 137.847 63.769002) (end 132.210984 58.132986) (width 0.3) (layer F.Cu) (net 4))
 (segment (start 132.210984 58.132986) (end 131.397016 58.132986) (width 0.3) (layer F.Cu) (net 4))
 (segment (start 130.347 59.183002) (end 131.397016 58.132986) (width 0.3) (layer B.Cu) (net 4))
 (via (at 131.397016 58.132986) (size 0.8) (drill 0.4) (layers F.Cu B.Cu) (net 4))
 (segment (start 86.947 64.693002) (end 86.947 63.033002) (width 0.3) (layer F.Cu) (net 4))
 (segment (start 86.947 63.033002) (end 91.847016 58.132986) (width 0.3) (layer F.Cu) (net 4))
 (segment (start 91.847016 58.132986) (end 131.397016 58.132986) (width 0.3) (layer F.Cu) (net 4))
 (via (at 94.162 49.929002) (size 0.8) (drill 0.4) (layers F.Cu B.Cu) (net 22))
 (segment (start 97.347 53.114002) (end 97.347 62.883002) (width 0.3) (layer B.Cu) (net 22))
 (segment (start 94.162 49.929002) (end 97.347 53.114002) (width 0.3) (layer B.Cu) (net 22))
 (segment (start 90.352 51.933002) (end 91.622 51.933002) (width 0.3) (layer F.Cu) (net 22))
 (segment (start 91.622 51.933002) (end 92.892 51.933002) (width 0.3) (layer F.Cu) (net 22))
 (segment (start 94.162 51.933002) (end 92.892 51.933002) (width 0.3) (layer F.Cu) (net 22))
 (segment (start 94.162 51.933002) (end 94.162 49.929002) (width 0.3) (layer F.Cu) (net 22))
 (via (at 104.322 49.929002) (size 0.8) (drill 0.4) (layers F.Cu B.Cu) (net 17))
 (segment (start 104.322 52.056) (end 104.322 49.929002) (width 0.3) (layer F.Cu) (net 17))
 (segment (start 105.597 51.204002) (end 105.597 62.883002) (width 0.3) (layer B.Cu) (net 17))
 (segment (start 104.322 49.929002) (end 105.597 51.204002) (width 0.3) (layer B.Cu) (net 17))
 (segment (start 100.512 51.933002) (end 101.782 51.933002) (width 0.3) (layer F.Cu) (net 17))
 (segment (start 101.782 51.933002) (end 103.052 51.933002) (width 0.3) (layer F.Cu) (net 17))
 (segment (start 103.052 51.933002) (end 104.322 51.933002) (width 0.3) (layer F.Cu) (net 17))
 (via (at 113.212 49.929002) (size 0.8) (drill 0.4) (layers F.Cu B.Cu) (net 11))
 (segment (start 113.212 52.056) (end 113.212 49.929002) (width 0.3) (layer F.Cu) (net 11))
 (segment (start 113.847 50.564002) (end 113.847 62.883002) (width 0.3) (layer B.Cu) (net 11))
 (segment (start 113.212 49.929002) (end 113.847 50.564002) (width 0.3) (layer B.Cu) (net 11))
 (segment (start 111.942 51.933002) (end 113.212 51.933002) (width 0.3) (layer F.Cu) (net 11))
 (segment (start 113.212 51.933002) (end 114.482 51.933002) (width 0.3) (layer F.Cu) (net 11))
 (segment (start 114.482 51.933002) (end 115.752 51.933002) (width 0.3) (layer F.Cu) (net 11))
 (via (at 133.347 55.383002) (size 0.8) (drill 0.4) (layers F.Cu B.Cu) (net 2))
 (segment (start 133.347 55.383002) (end 134.587 55.383002) (width 0.3) (layer F.Cu) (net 2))
 (segment (start 132.797 54.833002) (end 132.797 46.383002) (width 0.3) (layer B.Cu) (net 2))
 (segment (start 133.347 55.383002) (end 132.797 54.833002) (width 0.3) (layer B.Cu) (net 2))
 (via (at 135.597 57.133002) (size 0.8) (drill 0.4) (layers F.Cu B.Cu) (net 3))
 (segment (start 135.607 57.123002) (end 135.597 57.133002) (width 0.3) (layer F.Cu) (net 3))
 (segment (start 135.607 56.383002) (end 135.607 57.123002) (width 0.3) (layer F.Cu) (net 3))
 (segment (start 135.597 46.583002) (end 135.397 46.383002) (width 0.3) (layer B.Cu) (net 3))
 (segment (start 135.597 57.133002) (end 135.597 46.583002) (width 0.3) (layer B.Cu) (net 3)))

